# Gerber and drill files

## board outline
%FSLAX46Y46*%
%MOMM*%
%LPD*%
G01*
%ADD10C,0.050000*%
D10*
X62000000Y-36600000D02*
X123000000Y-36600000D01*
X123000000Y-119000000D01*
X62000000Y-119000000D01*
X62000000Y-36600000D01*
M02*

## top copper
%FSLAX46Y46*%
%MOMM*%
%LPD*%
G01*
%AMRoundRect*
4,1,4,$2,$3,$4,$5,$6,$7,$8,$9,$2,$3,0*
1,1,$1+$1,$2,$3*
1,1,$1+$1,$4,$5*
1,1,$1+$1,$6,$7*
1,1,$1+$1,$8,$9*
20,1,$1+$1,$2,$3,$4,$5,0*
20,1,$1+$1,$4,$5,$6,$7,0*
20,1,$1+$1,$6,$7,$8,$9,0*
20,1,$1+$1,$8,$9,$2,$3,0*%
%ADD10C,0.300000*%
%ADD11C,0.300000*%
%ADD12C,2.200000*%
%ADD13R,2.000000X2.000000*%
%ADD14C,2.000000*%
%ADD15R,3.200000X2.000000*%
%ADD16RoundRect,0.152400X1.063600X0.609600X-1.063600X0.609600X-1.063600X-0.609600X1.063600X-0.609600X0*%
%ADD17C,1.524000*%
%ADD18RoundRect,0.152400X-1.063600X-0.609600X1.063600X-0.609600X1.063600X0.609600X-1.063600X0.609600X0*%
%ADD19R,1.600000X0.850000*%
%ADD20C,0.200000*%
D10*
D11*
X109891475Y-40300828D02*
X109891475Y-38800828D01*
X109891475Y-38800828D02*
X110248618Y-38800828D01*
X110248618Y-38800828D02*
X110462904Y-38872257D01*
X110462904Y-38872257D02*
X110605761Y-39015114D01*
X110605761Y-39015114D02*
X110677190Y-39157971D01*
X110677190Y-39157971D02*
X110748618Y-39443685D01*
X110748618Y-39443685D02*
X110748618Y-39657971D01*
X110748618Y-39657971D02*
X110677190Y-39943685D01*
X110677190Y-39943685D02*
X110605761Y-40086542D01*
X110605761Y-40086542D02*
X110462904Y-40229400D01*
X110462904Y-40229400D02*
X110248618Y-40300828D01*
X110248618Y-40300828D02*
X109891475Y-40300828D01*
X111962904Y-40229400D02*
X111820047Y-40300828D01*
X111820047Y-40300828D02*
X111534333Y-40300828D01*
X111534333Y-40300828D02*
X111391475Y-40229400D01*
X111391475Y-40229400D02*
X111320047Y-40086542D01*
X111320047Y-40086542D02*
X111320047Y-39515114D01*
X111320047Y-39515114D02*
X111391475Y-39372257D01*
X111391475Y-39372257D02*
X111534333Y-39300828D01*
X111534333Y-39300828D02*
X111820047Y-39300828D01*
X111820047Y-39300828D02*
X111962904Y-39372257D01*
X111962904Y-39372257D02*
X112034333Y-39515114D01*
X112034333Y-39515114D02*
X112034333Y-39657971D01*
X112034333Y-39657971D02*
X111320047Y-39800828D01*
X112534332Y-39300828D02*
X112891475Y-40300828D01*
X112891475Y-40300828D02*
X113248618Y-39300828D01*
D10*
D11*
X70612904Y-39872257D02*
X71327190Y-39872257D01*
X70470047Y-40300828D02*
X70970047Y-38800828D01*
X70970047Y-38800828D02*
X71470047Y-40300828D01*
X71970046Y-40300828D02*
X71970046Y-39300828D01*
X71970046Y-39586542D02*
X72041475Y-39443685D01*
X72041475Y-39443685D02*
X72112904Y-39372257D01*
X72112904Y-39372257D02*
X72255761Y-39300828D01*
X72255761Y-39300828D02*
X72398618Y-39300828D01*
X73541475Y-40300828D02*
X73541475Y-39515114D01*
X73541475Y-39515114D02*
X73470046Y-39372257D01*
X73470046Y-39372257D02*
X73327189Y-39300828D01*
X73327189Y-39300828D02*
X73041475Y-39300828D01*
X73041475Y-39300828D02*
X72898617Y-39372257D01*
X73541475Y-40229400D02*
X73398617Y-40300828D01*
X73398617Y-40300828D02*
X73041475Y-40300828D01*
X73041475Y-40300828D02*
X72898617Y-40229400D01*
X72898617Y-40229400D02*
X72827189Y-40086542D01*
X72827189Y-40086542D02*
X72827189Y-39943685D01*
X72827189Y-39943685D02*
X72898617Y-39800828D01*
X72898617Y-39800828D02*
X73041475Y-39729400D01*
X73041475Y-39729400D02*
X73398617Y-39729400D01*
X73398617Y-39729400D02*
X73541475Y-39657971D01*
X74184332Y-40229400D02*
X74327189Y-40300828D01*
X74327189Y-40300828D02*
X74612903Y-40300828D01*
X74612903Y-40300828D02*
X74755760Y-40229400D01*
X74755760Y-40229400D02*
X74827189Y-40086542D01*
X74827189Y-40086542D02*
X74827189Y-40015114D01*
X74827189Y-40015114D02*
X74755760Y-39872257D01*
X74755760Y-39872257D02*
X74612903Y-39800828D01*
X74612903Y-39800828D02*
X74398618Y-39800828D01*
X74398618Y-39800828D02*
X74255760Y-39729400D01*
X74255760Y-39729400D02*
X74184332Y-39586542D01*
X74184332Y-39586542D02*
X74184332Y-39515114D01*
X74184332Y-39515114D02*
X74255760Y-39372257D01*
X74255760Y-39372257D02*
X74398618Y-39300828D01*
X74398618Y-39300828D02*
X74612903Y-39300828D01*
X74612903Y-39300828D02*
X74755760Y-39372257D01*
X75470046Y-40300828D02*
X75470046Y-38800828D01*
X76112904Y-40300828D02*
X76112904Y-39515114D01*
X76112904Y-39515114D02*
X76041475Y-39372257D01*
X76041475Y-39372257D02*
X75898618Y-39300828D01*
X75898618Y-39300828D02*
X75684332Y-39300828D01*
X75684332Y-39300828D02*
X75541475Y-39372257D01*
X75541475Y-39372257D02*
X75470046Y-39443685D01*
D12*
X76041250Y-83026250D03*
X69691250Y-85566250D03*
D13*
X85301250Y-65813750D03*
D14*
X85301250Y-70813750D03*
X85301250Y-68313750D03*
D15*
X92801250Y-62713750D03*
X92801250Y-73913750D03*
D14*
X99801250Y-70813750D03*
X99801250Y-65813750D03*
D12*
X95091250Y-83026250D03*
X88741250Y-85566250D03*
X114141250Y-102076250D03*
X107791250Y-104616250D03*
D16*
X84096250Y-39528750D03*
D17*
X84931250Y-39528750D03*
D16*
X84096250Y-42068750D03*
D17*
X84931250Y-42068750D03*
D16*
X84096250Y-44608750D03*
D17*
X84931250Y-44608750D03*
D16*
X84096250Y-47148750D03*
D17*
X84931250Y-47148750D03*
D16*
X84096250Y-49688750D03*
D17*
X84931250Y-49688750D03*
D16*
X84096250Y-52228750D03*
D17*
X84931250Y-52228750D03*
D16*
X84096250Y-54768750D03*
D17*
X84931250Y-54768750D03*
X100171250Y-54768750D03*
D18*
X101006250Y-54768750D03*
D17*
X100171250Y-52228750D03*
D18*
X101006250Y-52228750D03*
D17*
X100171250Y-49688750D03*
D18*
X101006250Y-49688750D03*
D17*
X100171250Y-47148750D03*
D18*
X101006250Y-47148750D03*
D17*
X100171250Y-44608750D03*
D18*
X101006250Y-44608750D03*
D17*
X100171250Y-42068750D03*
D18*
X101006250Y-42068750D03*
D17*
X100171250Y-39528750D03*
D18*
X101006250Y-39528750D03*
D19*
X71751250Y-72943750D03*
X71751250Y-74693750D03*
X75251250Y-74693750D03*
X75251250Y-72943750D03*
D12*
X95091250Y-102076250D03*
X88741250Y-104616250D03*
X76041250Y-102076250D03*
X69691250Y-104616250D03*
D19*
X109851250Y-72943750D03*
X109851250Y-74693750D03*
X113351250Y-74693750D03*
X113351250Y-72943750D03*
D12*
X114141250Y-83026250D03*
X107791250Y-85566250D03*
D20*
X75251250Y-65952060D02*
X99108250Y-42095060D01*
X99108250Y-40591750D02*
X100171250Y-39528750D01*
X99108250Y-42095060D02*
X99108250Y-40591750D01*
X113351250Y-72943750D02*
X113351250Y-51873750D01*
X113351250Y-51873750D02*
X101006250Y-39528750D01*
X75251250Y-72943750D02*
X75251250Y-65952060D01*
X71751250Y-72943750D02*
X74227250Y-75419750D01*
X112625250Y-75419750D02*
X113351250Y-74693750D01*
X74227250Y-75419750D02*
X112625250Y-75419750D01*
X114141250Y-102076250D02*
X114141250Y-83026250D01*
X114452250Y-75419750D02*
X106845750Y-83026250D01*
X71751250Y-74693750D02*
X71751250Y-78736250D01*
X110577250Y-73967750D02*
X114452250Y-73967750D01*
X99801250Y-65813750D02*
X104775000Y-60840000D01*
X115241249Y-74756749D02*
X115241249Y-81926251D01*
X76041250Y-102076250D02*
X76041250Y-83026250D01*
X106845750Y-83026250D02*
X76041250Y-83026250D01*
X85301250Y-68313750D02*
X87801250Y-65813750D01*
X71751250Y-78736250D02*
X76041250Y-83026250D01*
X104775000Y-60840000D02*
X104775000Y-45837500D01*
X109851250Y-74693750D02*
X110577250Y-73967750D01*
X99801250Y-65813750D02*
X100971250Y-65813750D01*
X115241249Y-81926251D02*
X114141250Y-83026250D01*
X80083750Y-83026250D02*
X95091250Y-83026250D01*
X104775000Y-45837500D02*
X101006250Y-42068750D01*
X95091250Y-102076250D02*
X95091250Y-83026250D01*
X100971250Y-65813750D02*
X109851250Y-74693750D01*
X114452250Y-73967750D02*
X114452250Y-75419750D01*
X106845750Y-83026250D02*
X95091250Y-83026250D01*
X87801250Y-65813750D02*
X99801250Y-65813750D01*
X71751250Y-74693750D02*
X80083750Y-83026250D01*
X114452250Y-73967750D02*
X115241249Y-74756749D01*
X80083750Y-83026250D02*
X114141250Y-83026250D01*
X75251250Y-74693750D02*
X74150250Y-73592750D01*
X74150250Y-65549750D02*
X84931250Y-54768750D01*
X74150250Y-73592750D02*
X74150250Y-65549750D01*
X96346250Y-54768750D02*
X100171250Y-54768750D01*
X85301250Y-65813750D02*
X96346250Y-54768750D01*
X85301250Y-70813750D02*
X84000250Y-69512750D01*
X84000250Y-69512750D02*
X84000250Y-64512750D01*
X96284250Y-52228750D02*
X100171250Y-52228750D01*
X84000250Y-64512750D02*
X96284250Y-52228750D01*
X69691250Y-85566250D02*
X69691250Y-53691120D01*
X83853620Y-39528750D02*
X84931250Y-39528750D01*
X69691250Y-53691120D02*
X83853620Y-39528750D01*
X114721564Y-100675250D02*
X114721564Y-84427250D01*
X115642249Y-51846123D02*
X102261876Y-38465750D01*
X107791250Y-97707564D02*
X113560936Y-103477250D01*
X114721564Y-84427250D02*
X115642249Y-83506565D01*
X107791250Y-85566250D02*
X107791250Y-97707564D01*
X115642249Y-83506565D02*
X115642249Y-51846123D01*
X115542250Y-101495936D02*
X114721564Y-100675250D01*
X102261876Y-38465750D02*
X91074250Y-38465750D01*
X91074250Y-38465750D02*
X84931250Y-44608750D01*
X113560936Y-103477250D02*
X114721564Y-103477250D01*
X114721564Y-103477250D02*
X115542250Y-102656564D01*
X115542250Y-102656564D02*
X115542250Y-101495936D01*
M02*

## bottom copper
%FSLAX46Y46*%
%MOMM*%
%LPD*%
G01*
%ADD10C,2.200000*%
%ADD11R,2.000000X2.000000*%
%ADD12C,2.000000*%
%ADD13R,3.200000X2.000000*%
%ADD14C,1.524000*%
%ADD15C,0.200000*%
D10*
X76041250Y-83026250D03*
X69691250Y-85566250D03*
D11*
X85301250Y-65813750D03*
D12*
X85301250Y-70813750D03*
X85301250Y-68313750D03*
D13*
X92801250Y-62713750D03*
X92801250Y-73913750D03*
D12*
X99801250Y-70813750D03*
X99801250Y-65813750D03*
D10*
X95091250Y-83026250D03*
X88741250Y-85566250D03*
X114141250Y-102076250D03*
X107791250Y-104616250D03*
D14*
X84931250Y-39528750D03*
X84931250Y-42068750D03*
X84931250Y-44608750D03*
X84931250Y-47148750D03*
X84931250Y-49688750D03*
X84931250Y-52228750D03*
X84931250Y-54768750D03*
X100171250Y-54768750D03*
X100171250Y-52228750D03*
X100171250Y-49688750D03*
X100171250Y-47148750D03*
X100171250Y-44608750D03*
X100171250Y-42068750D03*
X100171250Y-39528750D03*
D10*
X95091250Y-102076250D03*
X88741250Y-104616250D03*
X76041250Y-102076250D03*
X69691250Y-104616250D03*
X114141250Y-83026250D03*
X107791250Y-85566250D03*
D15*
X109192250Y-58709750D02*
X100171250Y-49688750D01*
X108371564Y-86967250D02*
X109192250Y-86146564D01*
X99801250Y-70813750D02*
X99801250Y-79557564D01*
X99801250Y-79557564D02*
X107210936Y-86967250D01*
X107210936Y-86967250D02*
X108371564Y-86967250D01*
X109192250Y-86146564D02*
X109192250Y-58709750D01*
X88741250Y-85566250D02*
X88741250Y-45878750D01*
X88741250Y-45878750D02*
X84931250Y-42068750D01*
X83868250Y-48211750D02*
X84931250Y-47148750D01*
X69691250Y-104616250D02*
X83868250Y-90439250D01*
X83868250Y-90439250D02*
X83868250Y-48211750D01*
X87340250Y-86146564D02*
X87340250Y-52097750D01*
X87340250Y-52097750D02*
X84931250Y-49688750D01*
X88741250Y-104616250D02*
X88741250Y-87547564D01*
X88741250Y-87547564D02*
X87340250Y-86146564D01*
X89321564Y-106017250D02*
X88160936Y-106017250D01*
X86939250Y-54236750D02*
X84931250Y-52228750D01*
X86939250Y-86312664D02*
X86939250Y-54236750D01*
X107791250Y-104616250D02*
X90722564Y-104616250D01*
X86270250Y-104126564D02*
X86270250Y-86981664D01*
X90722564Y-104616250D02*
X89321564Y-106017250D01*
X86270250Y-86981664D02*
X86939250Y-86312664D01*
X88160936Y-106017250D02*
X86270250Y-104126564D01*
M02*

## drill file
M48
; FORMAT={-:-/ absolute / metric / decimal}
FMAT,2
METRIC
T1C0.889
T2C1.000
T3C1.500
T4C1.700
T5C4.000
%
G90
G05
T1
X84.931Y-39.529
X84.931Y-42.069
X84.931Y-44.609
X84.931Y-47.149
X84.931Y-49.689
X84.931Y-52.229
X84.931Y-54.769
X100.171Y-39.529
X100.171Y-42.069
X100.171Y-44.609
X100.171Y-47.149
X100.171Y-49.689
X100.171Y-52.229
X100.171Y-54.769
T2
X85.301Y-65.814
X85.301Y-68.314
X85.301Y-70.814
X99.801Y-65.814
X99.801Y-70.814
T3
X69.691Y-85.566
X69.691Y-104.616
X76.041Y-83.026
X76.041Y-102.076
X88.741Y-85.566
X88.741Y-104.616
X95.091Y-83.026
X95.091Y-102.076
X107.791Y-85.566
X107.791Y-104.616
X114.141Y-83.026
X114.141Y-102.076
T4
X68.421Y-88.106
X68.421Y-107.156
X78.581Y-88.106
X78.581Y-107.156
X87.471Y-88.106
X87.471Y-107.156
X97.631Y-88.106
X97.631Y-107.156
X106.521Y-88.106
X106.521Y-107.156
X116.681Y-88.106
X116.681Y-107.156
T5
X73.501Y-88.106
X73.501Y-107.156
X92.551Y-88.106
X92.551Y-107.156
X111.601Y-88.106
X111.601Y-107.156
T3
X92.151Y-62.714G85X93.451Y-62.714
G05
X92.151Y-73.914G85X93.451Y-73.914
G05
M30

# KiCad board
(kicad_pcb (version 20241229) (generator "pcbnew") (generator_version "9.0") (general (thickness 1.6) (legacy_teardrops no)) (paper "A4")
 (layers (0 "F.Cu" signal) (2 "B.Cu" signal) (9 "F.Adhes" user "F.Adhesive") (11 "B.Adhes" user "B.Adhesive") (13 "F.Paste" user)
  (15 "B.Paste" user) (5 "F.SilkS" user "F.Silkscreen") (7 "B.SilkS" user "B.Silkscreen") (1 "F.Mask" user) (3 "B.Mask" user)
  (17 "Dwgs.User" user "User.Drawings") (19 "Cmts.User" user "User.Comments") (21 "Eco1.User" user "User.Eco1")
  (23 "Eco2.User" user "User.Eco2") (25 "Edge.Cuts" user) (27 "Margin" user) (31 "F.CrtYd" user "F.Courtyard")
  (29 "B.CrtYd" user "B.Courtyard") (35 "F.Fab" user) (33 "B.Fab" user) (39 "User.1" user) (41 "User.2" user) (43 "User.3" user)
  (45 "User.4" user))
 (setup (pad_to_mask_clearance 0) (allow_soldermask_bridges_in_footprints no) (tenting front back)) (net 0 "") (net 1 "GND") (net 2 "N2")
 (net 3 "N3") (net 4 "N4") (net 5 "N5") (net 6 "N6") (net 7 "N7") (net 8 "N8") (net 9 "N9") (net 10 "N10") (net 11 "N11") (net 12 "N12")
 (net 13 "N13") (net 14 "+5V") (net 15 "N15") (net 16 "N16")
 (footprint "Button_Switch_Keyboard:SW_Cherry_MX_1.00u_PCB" (layer "F.Cu") (at 76.04125 83.02625)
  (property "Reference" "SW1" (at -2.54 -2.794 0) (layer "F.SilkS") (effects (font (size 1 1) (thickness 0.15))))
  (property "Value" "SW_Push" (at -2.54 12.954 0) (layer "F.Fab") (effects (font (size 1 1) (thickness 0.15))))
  (pad "" np_thru_hole circle (at -7.62 5.08) (size 1.7 1.7) (drill 1.7) (layers "*.Cu" "*.Mask"))
  (pad "" np_thru_hole circle (at -2.54 5.08) (size 4 4) (drill 4) (layers "*.Cu" "*.Mask"))
  (pad "" np_thru_hole circle (at 2.54 5.08) (size 1.7 1.7) (drill 1.7) (layers "*.Cu" "*.Mask"))
  (pad "1" thru_hole circle (at 0 0) (size 2.2 2.2) (drill 1.5) (layers "*.Cu" "*.Mask") (remove_unused_layers no) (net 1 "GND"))
  (pad "2" thru_hole circle (at -6.35 2.54) (size 2.2 2.2) (drill 1.5) (layers "*.Cu" "*.Mask") (remove_unused_layers no) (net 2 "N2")))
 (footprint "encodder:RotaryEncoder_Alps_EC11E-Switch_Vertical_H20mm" (layer "F.Cu") (at 85.30125 65.81375)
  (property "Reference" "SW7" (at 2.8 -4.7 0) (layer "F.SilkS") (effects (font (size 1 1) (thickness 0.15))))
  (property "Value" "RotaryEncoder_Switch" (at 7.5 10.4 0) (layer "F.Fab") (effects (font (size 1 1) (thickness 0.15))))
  (pad "A" thru_hole rect (at 0 0) (size 2 2) (drill 1) (layers "*.Cu" "*.Mask") (remove_unused_layers no) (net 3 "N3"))
  (pad "B" thru_hole circle (at 0 5) (size 2 2) (drill 1) (layers "*.Cu" "*.Mask") (remove_unused_layers no) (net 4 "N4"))
  (pad "C" thru_hole circle (at 0 2.5) (size 2 2) (drill 1) (layers "*.Cu" "*.Mask") (remove_unused_layers no) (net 1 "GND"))
  (pad "MP" thru_hole rect (at 7.5 -3.1) (size 3.2 2) (drill oval 2.8 1.5) (layers "*.Cu" "*.Mask") (remove_unused_layers no))
  (pad "MP" thru_hole rect (at 7.5 8.1) (size 3.2 2) (drill oval 2.8 1.5) (layers "*.Cu" "*.Mask") (remove_unused_layers no))
  (pad "S1" thru_hole circle (at 14.5 5) (size 2 2) (drill 1) (layers "*.Cu" "*.Mask") (remove_unused_layers no) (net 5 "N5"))
  (pad "S2" thru_hole circle (at 14.5 0) (size 2 2) (drill 1) (layers "*.Cu" "*.Mask") (remove_unused_layers no) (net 1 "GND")))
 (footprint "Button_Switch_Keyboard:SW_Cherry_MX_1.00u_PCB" (layer "F.Cu") (at 95.09125 83.02625)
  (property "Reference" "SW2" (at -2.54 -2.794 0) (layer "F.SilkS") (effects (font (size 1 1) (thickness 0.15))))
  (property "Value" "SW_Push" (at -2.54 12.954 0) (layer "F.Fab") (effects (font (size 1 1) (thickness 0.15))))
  (pad "" np_thru_hole circle (at -7.62 5.08) (size 1.7 1.7) (drill 1.7) (layers "*.Cu" "*.Mask"))
  (pad "" np_thru_hole circle (at -2.54 5.08) (size 4 4) (drill 4) (layers "*.Cu" "*.Mask"))
  (pad "" np_thru_hole circle (at 2.54 5.08) (size 1.7 1.7) (drill 1.7) (layers "*.Cu" "*.Mask"))
  (pad "1" thru_hole circle (at 0 0) (size 2.2 2.2) (drill 1.5) (layers "*.Cu" "*.Mask") (remove_unused_layers no) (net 1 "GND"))
  (pad "2" thru_hole circle (at -6.35 2.54) (size 2.2 2.2) (drill 1.5) (layers "*.Cu" "*.Mask") (remove_unused_layers no) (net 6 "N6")))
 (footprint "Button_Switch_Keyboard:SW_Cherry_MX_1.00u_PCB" (layer "F.Cu") (at 114.14125 102.07625)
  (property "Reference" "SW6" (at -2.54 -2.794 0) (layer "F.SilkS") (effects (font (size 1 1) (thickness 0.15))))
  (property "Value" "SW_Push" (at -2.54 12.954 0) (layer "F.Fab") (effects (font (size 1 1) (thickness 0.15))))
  (pad "" np_thru_hole circle (at -7.62 5.08) (size 1.7 1.7) (drill 1.7) (layers "*.Cu" "*.Mask"))
  (pad "" np_thru_hole circle (at -2.54 5.08) (size 4 4) (drill 4) (layers "*.Cu" "*.Mask"))
  (pad "" np_thru_hole circle (at 2.54 5.08) (size 1.7 1.7) (drill 1.7) (layers "*.Cu" "*.Mask"))
  (pad "1" thru_hole circle (at 0 0) (size 2.2 2.2) (drill 1.5) (layers "*.Cu" "*.Mask") (remove_unused_layers no) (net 1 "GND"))
  (pad "2" thru_hole circle (at -6.35 2.54) (size 2.2 2.2) (drill 1.5) (layers "*.Cu" "*.Mask") (remove_unused_layers no) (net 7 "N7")))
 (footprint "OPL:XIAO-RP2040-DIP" (layer "F.Cu") (at 92.55125 47.14875)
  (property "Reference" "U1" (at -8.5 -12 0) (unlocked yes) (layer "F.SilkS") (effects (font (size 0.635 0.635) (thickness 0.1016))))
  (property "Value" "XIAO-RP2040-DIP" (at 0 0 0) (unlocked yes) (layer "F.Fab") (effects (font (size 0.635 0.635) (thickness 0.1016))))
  (pad "1" smd roundrect (at -8.455 -7.62 180) (size 2.432 1.524) (layers "F.Cu" "F.Mask") (roundrect_rratio 0.1) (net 2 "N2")
   (thermal_bridge_angle 45))
  (pad "1" thru_hole circle (at -7.62 -7.62 180) (size 1.524 1.524) (drill 0.889) (layers "*.Cu" "*.Mask") (remove_unused_layers no)
   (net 2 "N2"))
  (pad "2" smd roundrect (at -8.455 -5.08 180) (size 2.432 1.524) (layers "F.Cu" "F.Mask") (roundrect_rratio 0.1) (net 6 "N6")
   (thermal_bridge_angle 45))
  (pad "2" thru_hole circle (at -7.62 -5.08 180) (size 1.524 1.524) (drill 0.889) (layers "*.Cu" "*.Mask") (remove_unused_layers no)
   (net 6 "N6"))
  (pad "3" smd roundrect (at -8.455 -2.54 180) (size 2.432 1.524) (layers "F.Cu" "F.Mask") (roundrect_rratio 0.1) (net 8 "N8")
   (thermal_bridge_angle 45))
  (pad "3" thru_hole circle (at -7.62 -2.54 180) (size 1.524 1.524) (drill 0.889) (layers "*.Cu" "*.Mask") (remove_unused_layers no)
   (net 8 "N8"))
  (pad "4" smd roundrect (at -8.455 0 180) (size 2.432 1.524) (layers "F.Cu" "F.Mask") (roundrect_rratio 0.1) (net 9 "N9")
   (thermal_bridge_angle 45))
  (pad "4" thru_hole circle (at -7.62 0 180) (size 1.524 1.524) (drill 0.889) (layers "*.Cu" "*.Mask") (remove_unused_layers no)
   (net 9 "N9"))
  (pad "5" smd roundrect (at -8.455 2.54 180) (size 2.432 1.524) (layers "F.Cu" "F.Mask") (roundrect_rratio 0.1) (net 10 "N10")
   (thermal_bridge_angle 45))
  (pad "5" thru_hole circle (at -7.62 2.54 180) (size 1.524 1.524) (drill 0.889) (layers "*.Cu" "*.Mask") (remove_unused_layers no)
   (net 10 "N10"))
  (pad "6" smd roundrect (at -8.455 5.08 180) (size 2.432 1.524) (layers "F.Cu" "F.Mask") (roundrect_rratio 0.1) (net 7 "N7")
   (thermal_bridge_angle 45))
  (pad "6" thru_hole circle (at -7.62 5.08 180) (size 1.524 1.524) (drill 0.889) (layers "*.Cu" "*.Mask") (remove_unused_layers no)
   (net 7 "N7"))
  (pad "7" smd roundrect (at -8.455 7.62 180) (size 2.432 1.524) (layers "F.Cu" "F.Mask") (roundrect_rratio 0.1) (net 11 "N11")
   (thermal_bridge_angle 45))
  (pad "7" thru_hole circle (at -7.62 7.62 180) (size 1.524 1.524) (drill 0.889) (layers "*.Cu" "*.Mask") (remove_unused_layers no)
   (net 11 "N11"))
  (pad "8" thru_hole circle (at 7.62 7.62) (size 1.524 1.524) (drill 0.889) (layers "*.Cu" "*.Mask") (remove_unused_layers no) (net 3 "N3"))
  (pad "8" smd roundrect (at 8.455 7.62) (size 2.432 1.524) (layers "F.Cu" "F.Mask") (roundrect_rratio 0.1) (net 3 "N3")
   (thermal_bridge_angle 45))
  (pad "9" thru_hole circle (at 7.62 5.08) (size 1.524 1.524) (drill 0.889) (layers "*.Cu" "*.Mask") (remove_unused_layers no) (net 4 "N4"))
  (pad "9" smd roundrect (at 8.455 5.08) (size 2.432 1.524) (layers "F.Cu" "F.Mask") (roundrect_rratio 0.1) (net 4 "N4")
   (thermal_bridge_angle 45))
  (pad "10" thru_hole circle (at 7.62 2.54) (size 1.524 1.524) (drill 0.889) (layers "*.Cu" "*.Mask") (remove_unused_layers no) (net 5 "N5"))
  (pad "10" smd roundrect (at 8.455 2.54) (size 2.432 1.524) (layers "F.Cu" "F.Mask") (roundrect_rratio 0.1) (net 5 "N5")
   (thermal_bridge_angle 45))
  (pad "11" thru_hole circle (at 7.62 0) (size 1.524 1.524) (drill 0.889) (layers "*.Cu" "*.Mask") (remove_unused_layers no) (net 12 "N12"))
  (pad "11" smd roundrect (at 8.455 0) (size 2.432 1.524) (layers "F.Cu" "F.Mask") (roundrect_rratio 0.1) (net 12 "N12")
   (thermal_bridge_angle 45))
  (pad "12" thru_hole circle (at 7.62 -2.54) (size 1.524 1.524) (drill 0.889) (layers "*.Cu" "*.Mask") (remove_unused_layers no)
   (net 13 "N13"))
  (pad "12" smd roundrect (at 8.455 -2.54) (size 2.432 1.524) (layers "F.Cu" "F.Mask") (roundrect_rratio 0.1) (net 13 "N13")
   (thermal_bridge_angle 45))
  (pad "13" thru_hole circle (at 7.62 -5.08) (size 1.524 1.524) (drill 0.889) (layers "*.Cu" "*.Mask") (remove_unused_layers no)
   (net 1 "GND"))
  (pad "13" smd roundrect (at 8.455 -5.08) (size 2.432 1.524) (layers "F.Cu" "F.Mask") (roundrect_rratio 0.1) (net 1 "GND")
   (thermal_bridge_angle 45))
  (pad "14" thru_hole circle (at 7.62 -7.62) (size 1.524 1.524) (drill 0.889) (layers "*.Cu" "*.Mask") (remove_unused_layers no)
   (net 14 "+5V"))
  (pad "14" smd roundrect (at 8.455 -7.62) (size 2.432 1.524) (layers "F.Cu" "F.Mask") (roundrect_rratio 0.1) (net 14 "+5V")
   (thermal_bridge_angle 45)))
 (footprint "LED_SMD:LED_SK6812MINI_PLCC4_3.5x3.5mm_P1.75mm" (layer "F.Cu") (at 73.50125 73.81875)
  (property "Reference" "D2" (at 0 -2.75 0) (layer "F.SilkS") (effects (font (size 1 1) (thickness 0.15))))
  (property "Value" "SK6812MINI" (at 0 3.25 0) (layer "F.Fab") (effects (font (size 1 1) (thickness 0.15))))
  (pad "1" smd rect (at -1.75 -0.875) (size 1.6 0.85) (layers "F.Cu" "F.Mask" "F.Paste") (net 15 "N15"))
  (pad "2" smd rect (at -1.75 0.875) (size 1.6 0.85) (layers "F.Cu" "F.Mask" "F.Paste") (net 1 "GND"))
  (pad "3" smd rect (at 1.75 0.875) (size 1.6 0.85) (layers "F.Cu" "F.Mask" "F.Paste") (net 11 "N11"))
  (pad "4" smd rect (at 1.75 -0.875) (size 1.6 0.85) (layers "F.Cu" "F.Mask" "F.Paste") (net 14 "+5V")))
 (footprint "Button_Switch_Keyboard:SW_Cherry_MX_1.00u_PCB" (layer "F.Cu") (at 95.09125 102.07625)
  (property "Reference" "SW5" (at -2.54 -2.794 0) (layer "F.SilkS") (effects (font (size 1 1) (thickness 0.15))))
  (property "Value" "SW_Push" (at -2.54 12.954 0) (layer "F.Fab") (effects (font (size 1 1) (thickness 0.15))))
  (pad "" np_thru_hole circle (at -7.62 5.08) (size 1.7 1.7) (drill 1.7) (layers "*.Cu" "*.Mask"))
  (pad "" np_thru_hole circle (at -2.54 5.08) (size 4 4) (drill 4) (layers "*.Cu" "*.Mask"))
  (pad "" np_thru_hole circle (at 2.54 5.08) (size 1.7 1.7) (drill 1.7) (layers "*.Cu" "*.Mask"))
  (pad "1" thru_hole circle (at 0 0) (size 2.2 2.2) (drill 1.5) (layers "*.Cu" "*.Mask") (remove_unused_layers no) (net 1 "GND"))
  (pad "2" thru_hole circle (at -6.35 2.54) (size 2.2 2.2) (drill 1.5) (layers "*.Cu" "*.Mask") (remove_unused_layers no) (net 10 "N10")))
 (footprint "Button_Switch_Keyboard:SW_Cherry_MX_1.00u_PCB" (layer "F.Cu") (at 76.04125 102.07625)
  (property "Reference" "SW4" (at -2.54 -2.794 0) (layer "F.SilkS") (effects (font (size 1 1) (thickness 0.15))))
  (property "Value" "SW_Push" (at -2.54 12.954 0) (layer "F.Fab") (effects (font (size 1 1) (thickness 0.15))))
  (pad "" np_thru_hole circle (at -7.62 5.08) (size 1.7 1.7) (drill 1.7) (layers "*.Cu" "*.Mask"))
  (pad "" np_thru_hole circle (at -2.54 5.08) (size 4 4) (drill 4) (layers "*.Cu" "*.Mask"))
  (pad "" np_thru_hole circle (at 2.54 5.08) (size 1.7 1.7) (drill 1.7) (layers "*.Cu" "*.Mask"))
  (pad "1" thru_hole circle (at 0 0) (size 2.2 2.2) (drill 1.5) (layers "*.Cu" "*.Mask") (remove_unused_layers no) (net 1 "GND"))
  (pad "2" thru_hole circle (at -6.35 2.54) (size 2.2 2.2) (drill 1.5) (layers "*.Cu" "*.Mask") (remove_unused_layers no) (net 9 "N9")))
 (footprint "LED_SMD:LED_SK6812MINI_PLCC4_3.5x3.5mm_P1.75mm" (layer "F.Cu") (at 111.60125 73.81875)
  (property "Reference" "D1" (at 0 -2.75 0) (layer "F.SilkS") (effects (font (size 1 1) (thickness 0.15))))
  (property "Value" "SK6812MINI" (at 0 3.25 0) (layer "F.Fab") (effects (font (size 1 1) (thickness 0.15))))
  (pad "1" smd rect (at -1.75 -0.875) (size 1.6 0.85) (layers "F.Cu" "F.Mask" "F.Paste") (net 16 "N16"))
  (pad "2" smd rect (at -1.75 0.875) (size 1.6 0.85) (layers "F.Cu" "F.Mask" "F.Paste") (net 1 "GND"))
  (pad "3" smd rect (at 1.75 0.875) (size 1.6 0.85) (layers "F.Cu" "F.Mask" "F.Paste") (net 15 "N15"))
  (pad "4" smd rect (at 1.75 -0.875) (size 1.6 0.85) (layers "F.Cu" "F.Mask" "F.Paste") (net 14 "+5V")))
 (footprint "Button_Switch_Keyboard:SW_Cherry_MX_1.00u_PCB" (layer "F.Cu") (at 114.14125 83.02625)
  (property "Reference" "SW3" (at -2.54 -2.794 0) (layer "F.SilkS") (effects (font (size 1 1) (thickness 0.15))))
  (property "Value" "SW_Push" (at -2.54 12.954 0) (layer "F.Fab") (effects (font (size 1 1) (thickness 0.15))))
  (pad "" np_thru_hole circle (at -7.62 5.08) (size 1.7 1.7) (drill 1.7) (layers "*.Cu" "*.Mask"))
  (pad "" np_thru_hole circle (at -2.54 5.08) (size 4 4) (drill 4) (layers "*.Cu" "*.Mask"))
  (pad "" np_thru_hole circle (at 2.54 5.08) (size 1.7 1.7) (drill 1.7) (layers "*.Cu" "*.Mask"))
  (pad "1" thru_hole circle (at 0 0) (size 2.2 2.2) (drill 1.5) (layers "*.Cu" "*.Mask") (remove_unused_layers no) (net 1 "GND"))
  (pad "2" thru_hole circle (at -6.35 2.54) (size 2.2 2.2) (drill 1.5) (layers "*.Cu" "*.Mask") (remove_unused_layers no) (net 8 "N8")))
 (gr_rect (start 62 36.6) (end 123 119) (stroke (width 0.05) (type default)) (fill no) (layer "Edge.Cuts"))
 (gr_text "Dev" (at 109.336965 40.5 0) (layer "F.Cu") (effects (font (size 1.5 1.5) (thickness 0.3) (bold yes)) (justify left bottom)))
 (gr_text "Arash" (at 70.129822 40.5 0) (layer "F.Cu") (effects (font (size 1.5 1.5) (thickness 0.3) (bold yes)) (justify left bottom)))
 (segment (start 75.25125 65.95206) (end 99.10825 42.09506) (width 0.2) (layer "F.Cu") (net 14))
 (segment (start 99.10825 40.59175) (end 100.17125 39.52875) (width 0.2) (layer "F.Cu") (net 14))
 (segment (start 99.10825 42.09506) (end 99.10825 40.59175) (width 0.2) (layer "F.Cu") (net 14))
 (segment (start 113.35125 72.94375) (end 113.35125 51.87375) (width 0.2) (layer "F.Cu") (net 14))
 (segment (start 113.35125 51.87375) (end 101.00625 39.52875) (width 0.2) (layer "F.Cu") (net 14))
 (segment (start 75.25125 72.94375) (end 75.25125 65.95206) (width 0.2) (layer "F.Cu") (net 14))
 (segment (start 71.75125 72.94375) (end 74.22725 75.41975) (width 0.2) (layer "F.Cu") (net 15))
 (segment (start 112.62525 75.41975) (end 113.35125 74.69375) (width 0.2) (layer "F.Cu") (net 15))
 (segment (start 74.22725 75.41975) (end 112.62525 75.41975) (width 0.2) (layer "F.Cu") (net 15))
 (segment (start 114.14125 102.07625) (end 114.14125 83.02625) (width 0.2) (layer "F.Cu") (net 1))
 (segment (start 114.45225 75.41975) (end 106.84575 83.02625) (width 0.2) (layer "F.Cu") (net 1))
 (segment (start 71.75125 74.69375) (end 71.75125 78.73625) (width 0.2) (layer "F.Cu") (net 1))
 (segment (start 110.57725 73.96775) (end 114.45225 73.96775) (width 0.2) (layer "F.Cu") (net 1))
 (segment (start 99.80125 65.81375) (end 104.775 60.84) (width 0.2) (layer "F.Cu") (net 1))
 (segment (start 115.241249 74.756749) (end 115.241249 81.926251) (width 0.2) (layer "F.Cu") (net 1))
 (segment (start 76.04125 102.07625) (end 76.04125 83.02625) (width 0.2) (layer "F.Cu") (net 1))
 (segment (start 106.84575 83.02625) (end 76.04125 83.02625) (width 0.2) (layer "F.Cu") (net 1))
 (segment (start 85.30125 68.31375) (end 87.80125 65.81375) (width 0.2) (layer "F.Cu") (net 1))
 (segment (start 71.75125 78.73625) (end 76.04125 83.02625) (width 0.2) (layer "F.Cu") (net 1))
 (segment (start 104.775 60.84) (end 104.775 45.8375) (width 0.2) (layer "F.Cu") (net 1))
 (segment (start 109.85125 74.69375) (end 110.57725 73.96775) (width 0.2) (layer "F.Cu") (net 1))
 (segment (start 99.80125 65.81375) (end 100.97125 65.81375) (width 0.2) (layer "F.Cu") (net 1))
 (segment (start 115.241249 81.926251) (end 114.14125 83.02625) (width 0.2) (layer "F.Cu") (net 1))
 (segment (start 80.08375 83.02625) (end 95.09125 83.02625) (width 0.2) (layer "F.Cu") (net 1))
 (segment (start 104.775 45.8375) (end 101.00625 42.06875) (width 0.2) (layer "F.Cu") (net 1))
 (segment (start 95.09125 102.07625) (end 95.09125 83.02625) (width 0.2) (layer "F.Cu") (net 1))
 (segment (start 100.97125 65.81375) (end 109.85125 74.69375) (width 0.2) (layer "F.Cu") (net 1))
 (segment (start 114.45225 73.96775) (end 114.45225 75.41975) (width 0.2) (layer "F.Cu") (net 1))
 (segment (start 106.84575 83.02625) (end 95.09125 83.02625) (width 0.2) (layer "F.Cu") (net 1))
 (segment (start 87.80125 65.81375) (end 99.80125 65.81375) (width 0.2) (layer "F.Cu") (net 1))
 (segment (start 71.75125 74.69375) (end 80.08375 83.02625) (width 0.2) (layer "F.Cu") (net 1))
 (segment (start 114.45225 73.96775) (end 115.241249 74.756749) (width 0.2) (layer "F.Cu") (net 1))
 (segment (start 80.08375 83.02625) (end 114.14125 83.02625) (width 0.2) (layer "F.Cu") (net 1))
 (segment (start 75.25125 74.69375) (end 74.15025 73.59275) (width 0.2) (layer "F.Cu") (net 11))
 (segment (start 74.15025 65.54975) (end 84.93125 54.76875) (width 0.2) (layer "F.Cu") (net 11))
 (segment (start 74.15025 73.59275) (end 74.15025 65.54975) (width 0.2) (layer "F.Cu") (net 11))
 (segment (start 96.34625 54.76875) (end 100.17125 54.76875) (width 0.2) (layer "F.Cu") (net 3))
 (segment (start 85.30125 65.81375) (end 96.34625 54.76875) (width 0.2) (layer "F.Cu") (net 3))
 (segment (start 85.30125 70.81375) (end 84.00025 69.51275) (width 0.2) (layer "F.Cu") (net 4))
 (segment (start 84.00025 69.51275) (end 84.00025 64.51275) (width 0.2) (layer "F.Cu") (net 4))
 (segment (start 96.28425 52.22875) (end 100.17125 52.22875) (width 0.2) (layer "F.Cu") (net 4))
 (segment (start 84.00025 64.51275) (end 96.28425 52.22875) (width 0.2) (layer "F.Cu") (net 4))
 (segment (start 109.19225 58.70975) (end 100.17125 49.68875) (width 0.2) (layer "B.Cu") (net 5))
 (segment (start 108.371564 86.96725) (end 109.19225 86.146564) (width 0.2) (layer "B.Cu") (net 5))
 (segment (start 99.80125 70.81375) (end 99.80125 79.557564) (width 0.2) (layer "B.Cu") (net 5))
 (segment (start 99.80125 79.557564) (end 107.210936 86.96725) (width 0.2) (layer "B.Cu") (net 5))
 (segment (start 107.210936 86.96725) (end 108.371564 86.96725) (width 0.2) (layer "B.Cu") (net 5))
 (segment (start 109.19225 86.146564) (end 109.19225 58.70975) (width 0.2) (layer "B.Cu") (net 5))
 (segment (start 69.69125 85.56625) (end 69.69125 53.69112) (width 0.2) (layer "F.Cu") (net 2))
 (segment (start 83.85362 39.52875) (end 84.93125 39.52875) (width 0.2) (layer "F.Cu") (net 2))
 (segment (start 69.69125 53.69112) (end 83.85362 39.52875) (width 0.2) (layer "F.Cu") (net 2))
 (segment (start 88.74125 85.56625) (end 88.74125 45.87875) (width 0.2) (layer "B.Cu") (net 6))
 (segment (start 88.74125 45.87875) (end 84.93125 42.06875) (width 0.2) (layer "B.Cu") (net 6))
 (segment (start 114.721564 100.67525) (end 114.721564 84.42725) (width 0.2) (layer "F.Cu") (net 8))
 (segment (start 115.642249 51.846123) (end 102.261876 38.46575) (width 0.2) (layer "F.Cu") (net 8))
 (segment (start 107.79125 97.707564) (end 113.560936 103.47725) (width 0.2) (layer "F.Cu") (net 8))
 (segment (start 114.721564 84.42725) (end 115.642249 83.506565) (width 0.2) (layer "F.Cu") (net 8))
 (segment (start 107.79125 85.56625) (end 107.79125 97.707564) (width 0.2) (layer "F.Cu") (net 8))
 (segment (start 115.642249 83.506565) (end 115.642249 51.846123) (width 0.2) (layer "F.Cu") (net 8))
 (segment (start 115.54225 101.495936) (end 114.721564 100.67525) (width 0.2) (layer "F.Cu") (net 8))
 (segment (start 102.261876 38.46575) (end 91.07425 38.46575) (width 0.2) (layer "F.Cu") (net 8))
 (segment (start 91.07425 38.46575) (end 84.93125 44.60875) (width 0.2) (layer "F.Cu") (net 8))
 (segment (start 113.560936 103.47725) (end 114.721564 103.47725) (width 0.2) (layer "F.Cu") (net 8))
 (segment (start 114.721564 103.47725) (end 115.54225 102.656564) (width 0.2) (layer "F.Cu") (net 8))
 (segment (start 115.54225 102.656564) (end 115.54225 101.495936) (width 0.2) (layer "F.Cu") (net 8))
 (segment (start 83.86825 48.21175) (end 84.93125 47.14875) (width 0.2) (layer "B.Cu") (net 9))
 (segment (start 69.69125 104.61625) (end 83.86825 90.43925) (width 0.2) (layer "B.Cu") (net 9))
 (segment (start 83.86825 90.43925) (end 83.86825 48.21175) (width 0.2) (layer "B.Cu") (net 9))
 (segment (start 87.34025 86.146564) (end 87.34025 52.09775) (width 0.2) (layer "B.Cu") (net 10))
 (segment (start 87.34025 52.09775) (end 84.93125 49.68875) (width 0.2) (layer "B.Cu") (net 10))
 (segment (start 88.74125 104.61625) (end 88.74125 87.547564) (width 0.2) (layer "B.Cu") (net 10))
 (segment (start 88.74125 87.547564) (end 87.34025 86.146564) (width 0.2) (layer "B.Cu") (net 10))
 (segment (start 89.321564 106.01725) (end 88.160936 106.01725) (width 0.2) (layer "B.Cu") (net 7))
 (segment (start 86.93925 54.23675) (end 84.93125 52.22875) (width 0.2) (layer "B.Cu") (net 7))
 (segment (start 86.93925 86.312664) (end 86.93925 54.23675) (width 0.2) (layer "B.Cu") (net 7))
 (segment (start 107.79125 104.61625) (end 90.722564 104.61625) (width 0.2) (layer "B.Cu") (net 7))
 (segment (start 86.27025 104.126564) (end 86.27025 86.981664) (width 0.2) (layer "B.Cu") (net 7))
 (segment (start 90.722564 104.61625) (end 89.321564 106.01725) (width 0.2) (layer "B.Cu") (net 7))
 (segment (start 86.27025 86.981664) (end 86.93925 86.312664) (width 0.2) (layer "B.Cu") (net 7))
 (segment (start 88.160936 106.01725) (end 86.27025 104.126564) (width 0.2) (layer "B.Cu") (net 7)))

